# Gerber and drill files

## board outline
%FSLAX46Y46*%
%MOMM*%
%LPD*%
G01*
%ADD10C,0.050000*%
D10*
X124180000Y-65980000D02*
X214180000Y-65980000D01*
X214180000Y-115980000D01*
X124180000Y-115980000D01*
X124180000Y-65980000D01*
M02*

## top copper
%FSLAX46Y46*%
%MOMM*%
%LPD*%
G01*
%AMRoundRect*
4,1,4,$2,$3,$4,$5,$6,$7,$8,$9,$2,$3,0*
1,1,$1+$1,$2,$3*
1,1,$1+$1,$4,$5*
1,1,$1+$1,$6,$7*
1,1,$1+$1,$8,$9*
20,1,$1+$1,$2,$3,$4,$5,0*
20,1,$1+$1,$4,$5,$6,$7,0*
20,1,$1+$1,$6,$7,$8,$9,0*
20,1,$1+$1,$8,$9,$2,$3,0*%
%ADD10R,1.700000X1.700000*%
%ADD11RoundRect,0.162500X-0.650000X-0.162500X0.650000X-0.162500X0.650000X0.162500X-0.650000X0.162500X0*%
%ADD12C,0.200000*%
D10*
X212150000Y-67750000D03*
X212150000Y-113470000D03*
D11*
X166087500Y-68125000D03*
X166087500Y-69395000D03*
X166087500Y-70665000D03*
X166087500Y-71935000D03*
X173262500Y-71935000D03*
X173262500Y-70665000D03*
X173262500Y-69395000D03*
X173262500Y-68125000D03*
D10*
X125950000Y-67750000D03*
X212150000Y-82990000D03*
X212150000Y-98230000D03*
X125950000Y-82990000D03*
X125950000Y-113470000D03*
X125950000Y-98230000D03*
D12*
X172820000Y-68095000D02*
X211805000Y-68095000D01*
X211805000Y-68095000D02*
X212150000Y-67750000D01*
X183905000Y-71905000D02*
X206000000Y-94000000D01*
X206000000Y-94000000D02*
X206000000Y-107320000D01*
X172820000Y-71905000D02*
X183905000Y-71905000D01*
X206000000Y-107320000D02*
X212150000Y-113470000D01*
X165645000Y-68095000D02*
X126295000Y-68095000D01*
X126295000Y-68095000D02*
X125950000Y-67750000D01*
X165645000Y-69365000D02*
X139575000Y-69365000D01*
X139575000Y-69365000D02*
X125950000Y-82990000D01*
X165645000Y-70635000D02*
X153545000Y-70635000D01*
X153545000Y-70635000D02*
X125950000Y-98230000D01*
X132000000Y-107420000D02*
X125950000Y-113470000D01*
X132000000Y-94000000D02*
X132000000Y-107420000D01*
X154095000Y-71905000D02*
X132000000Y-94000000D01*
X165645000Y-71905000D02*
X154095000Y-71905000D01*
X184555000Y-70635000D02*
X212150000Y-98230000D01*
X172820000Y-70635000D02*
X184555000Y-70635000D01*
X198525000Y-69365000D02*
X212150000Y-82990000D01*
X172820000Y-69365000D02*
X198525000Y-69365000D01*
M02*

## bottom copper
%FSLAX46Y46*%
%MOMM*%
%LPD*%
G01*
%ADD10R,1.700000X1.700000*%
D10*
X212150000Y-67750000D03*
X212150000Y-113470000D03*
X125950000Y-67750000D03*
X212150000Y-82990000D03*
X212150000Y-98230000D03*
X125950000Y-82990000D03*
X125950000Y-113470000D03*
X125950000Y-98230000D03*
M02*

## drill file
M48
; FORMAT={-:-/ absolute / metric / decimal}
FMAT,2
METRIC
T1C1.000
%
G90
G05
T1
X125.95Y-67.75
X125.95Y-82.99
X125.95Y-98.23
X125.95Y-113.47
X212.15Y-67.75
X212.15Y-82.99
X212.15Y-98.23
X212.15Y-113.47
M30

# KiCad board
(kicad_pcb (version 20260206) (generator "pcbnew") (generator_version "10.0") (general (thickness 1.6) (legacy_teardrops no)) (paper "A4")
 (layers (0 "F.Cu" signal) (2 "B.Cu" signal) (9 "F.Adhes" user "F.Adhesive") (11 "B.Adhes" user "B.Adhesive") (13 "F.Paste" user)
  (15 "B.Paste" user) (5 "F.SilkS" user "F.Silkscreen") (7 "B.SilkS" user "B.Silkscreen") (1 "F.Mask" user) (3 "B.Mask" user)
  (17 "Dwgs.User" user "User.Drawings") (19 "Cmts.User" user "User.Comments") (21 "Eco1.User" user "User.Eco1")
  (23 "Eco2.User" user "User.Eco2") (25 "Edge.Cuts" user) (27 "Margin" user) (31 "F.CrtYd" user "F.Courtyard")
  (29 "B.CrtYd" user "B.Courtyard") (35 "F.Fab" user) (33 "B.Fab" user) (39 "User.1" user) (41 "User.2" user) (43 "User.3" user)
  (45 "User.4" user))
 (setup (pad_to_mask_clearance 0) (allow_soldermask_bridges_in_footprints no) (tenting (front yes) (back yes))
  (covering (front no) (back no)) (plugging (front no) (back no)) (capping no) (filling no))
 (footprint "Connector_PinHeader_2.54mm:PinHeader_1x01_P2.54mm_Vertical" (layer "F.Cu") (at 212.15 67.75)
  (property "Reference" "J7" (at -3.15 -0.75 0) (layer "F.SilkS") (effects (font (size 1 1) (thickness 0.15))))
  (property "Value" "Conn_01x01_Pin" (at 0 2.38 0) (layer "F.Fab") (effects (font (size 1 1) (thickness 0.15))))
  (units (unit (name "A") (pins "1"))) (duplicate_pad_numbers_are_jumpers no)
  (pad "1" thru_hole rect (at 0 0) (size 1.7 1.7) (drill 1) (layers "*.Cu" "*.Mask") (remove_unused_layers no) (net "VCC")))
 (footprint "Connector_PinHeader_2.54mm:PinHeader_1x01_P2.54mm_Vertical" (layer "F.Cu") (at 212.15 113.47)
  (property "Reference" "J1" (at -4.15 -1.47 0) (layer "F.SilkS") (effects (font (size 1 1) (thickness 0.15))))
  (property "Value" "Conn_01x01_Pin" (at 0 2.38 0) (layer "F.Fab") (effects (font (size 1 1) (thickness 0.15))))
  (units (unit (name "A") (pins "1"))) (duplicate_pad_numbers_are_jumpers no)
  (pad "1" thru_hole rect (at 0 0) (size 1.7 1.7) (drill 1) (layers "*.Cu" "*.Mask") (remove_unused_layers no) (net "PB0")))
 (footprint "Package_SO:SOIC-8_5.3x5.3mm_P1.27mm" (layer "F.Cu") (at 169.675 70.03)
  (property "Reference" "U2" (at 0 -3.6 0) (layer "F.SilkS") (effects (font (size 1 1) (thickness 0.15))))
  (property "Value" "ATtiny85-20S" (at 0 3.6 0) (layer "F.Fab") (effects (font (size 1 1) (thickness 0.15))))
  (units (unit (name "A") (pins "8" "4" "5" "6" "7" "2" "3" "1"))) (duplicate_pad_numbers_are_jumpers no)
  (pad "1" smd roundrect (at -3.5875 -1.905) (size 1.625 0.65) (layers "F.Cu" "F.Mask" "F.Paste") (roundrect_rratio 0.25) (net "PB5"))
  (pad "2" smd roundrect (at -3.5875 -0.635) (size 1.625 0.65) (layers "F.Cu" "F.Mask" "F.Paste") (roundrect_rratio 0.25) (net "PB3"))
  (pad "3" smd roundrect (at -3.5875 0.635) (size 1.625 0.65) (layers "F.Cu" "F.Mask" "F.Paste") (roundrect_rratio 0.25) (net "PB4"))
  (pad "4" smd roundrect (at -3.5875 1.905) (size 1.625 0.65) (layers "F.Cu" "F.Mask" "F.Paste") (roundrect_rratio 0.25) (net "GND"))
  (pad "5" smd roundrect (at 3.5875 1.905) (size 1.625 0.65) (layers "F.Cu" "F.Mask" "F.Paste") (roundrect_rratio 0.25) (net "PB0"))
  (pad "6" smd roundrect (at 3.5875 0.635) (size 1.625 0.65) (layers "F.Cu" "F.Mask" "F.Paste") (roundrect_rratio 0.25) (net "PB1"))
  (pad "7" smd roundrect (at 3.5875 -0.635) (size 1.625 0.65) (layers "F.Cu" "F.Mask" "F.Paste") (roundrect_rratio 0.25) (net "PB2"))
  (pad "8" smd roundrect (at 3.5875 -1.905) (size 1.625 0.65) (layers "F.Cu" "F.Mask" "F.Paste") (roundrect_rratio 0.25) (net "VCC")))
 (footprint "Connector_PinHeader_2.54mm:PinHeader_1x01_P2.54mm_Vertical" (layer "F.Cu") (at 125.95 67.75)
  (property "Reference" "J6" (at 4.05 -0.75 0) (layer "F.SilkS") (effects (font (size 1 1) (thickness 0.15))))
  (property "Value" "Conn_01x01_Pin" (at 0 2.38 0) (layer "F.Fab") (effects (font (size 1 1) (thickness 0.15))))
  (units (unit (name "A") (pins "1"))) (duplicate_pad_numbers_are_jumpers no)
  (pad "1" thru_hole rect (at 0 0) (size 1.7 1.7) (drill 1) (layers "*.Cu" "*.Mask") (remove_unused_layers no) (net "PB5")))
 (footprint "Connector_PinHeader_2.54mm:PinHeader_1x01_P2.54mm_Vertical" (layer "F.Cu") (at 212.15 82.99)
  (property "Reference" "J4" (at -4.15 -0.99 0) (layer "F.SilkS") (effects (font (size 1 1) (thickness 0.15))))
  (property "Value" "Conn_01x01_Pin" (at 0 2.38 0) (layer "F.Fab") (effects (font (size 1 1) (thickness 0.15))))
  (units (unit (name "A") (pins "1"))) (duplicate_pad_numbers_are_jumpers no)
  (pad "1" thru_hole rect (at 0 0) (size 1.7 1.7) (drill 1) (layers "*.Cu" "*.Mask") (remove_unused_layers no) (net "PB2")))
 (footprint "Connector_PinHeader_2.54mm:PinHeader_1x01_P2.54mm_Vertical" (layer "F.Cu") (at 212.15 98.23)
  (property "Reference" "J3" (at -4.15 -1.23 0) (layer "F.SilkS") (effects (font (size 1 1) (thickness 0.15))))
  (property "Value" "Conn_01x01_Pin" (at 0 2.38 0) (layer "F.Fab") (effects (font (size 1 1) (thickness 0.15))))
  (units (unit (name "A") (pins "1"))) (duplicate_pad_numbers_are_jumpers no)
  (pad "1" thru_hole rect (at 0 0) (size 1.7 1.7) (drill 1) (layers "*.Cu" "*.Mask") (remove_unused_layers no) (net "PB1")))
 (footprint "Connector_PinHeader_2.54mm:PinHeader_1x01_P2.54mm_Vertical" (layer "F.Cu") (at 125.95 82.99)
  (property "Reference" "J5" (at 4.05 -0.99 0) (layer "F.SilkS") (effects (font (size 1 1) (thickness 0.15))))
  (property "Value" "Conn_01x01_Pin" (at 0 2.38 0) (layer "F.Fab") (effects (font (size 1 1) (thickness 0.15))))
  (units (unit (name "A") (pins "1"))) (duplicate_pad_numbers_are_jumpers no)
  (pad "1" thru_hole rect (at 0 0) (size 1.7 1.7) (drill 1) (layers "*.Cu" "*.Mask") (remove_unused_layers no) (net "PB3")))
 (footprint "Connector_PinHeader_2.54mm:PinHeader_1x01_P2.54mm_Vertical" (layer "F.Cu") (at 125.95 113.47)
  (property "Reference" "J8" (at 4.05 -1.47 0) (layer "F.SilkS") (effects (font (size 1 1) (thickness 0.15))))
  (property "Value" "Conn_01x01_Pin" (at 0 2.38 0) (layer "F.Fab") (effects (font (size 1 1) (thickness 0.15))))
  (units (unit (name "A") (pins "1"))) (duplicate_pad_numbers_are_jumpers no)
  (pad "1" thru_hole rect (at 0 0) (size 1.7 1.7) (drill 1) (layers "*.Cu" "*.Mask") (remove_unused_layers no) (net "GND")))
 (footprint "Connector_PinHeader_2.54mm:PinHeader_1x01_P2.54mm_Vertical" (layer "F.Cu") (at 125.95 98.23)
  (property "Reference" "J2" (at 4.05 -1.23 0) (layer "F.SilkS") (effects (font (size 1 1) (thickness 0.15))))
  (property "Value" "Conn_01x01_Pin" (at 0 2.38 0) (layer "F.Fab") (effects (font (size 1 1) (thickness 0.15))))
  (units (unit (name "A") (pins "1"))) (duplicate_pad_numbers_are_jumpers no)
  (pad "1" thru_hole rect (at 0 0) (size 1.7 1.7) (drill 1) (layers "*.Cu" "*.Mask") (remove_unused_layers no) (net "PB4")))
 (gr_rect (start 124.18 65.98) (end 214.18 115.98) (stroke (width 0.05) (type default)) (fill no) (layer "Edge.Cuts"))
 (segment (start 172.82 68.095) (end 211.805 68.095) (width 0.2) (layer "F.Cu") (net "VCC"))
 (segment (start 211.805 68.095) (end 212.15 67.75) (width 0.2) (layer "F.Cu") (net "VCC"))
 (segment (start 183.905 71.905) (end 206 94) (width 0.2) (layer "F.Cu") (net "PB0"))
 (segment (start 206 94) (end 206 107.32) (width 0.2) (layer "F.Cu") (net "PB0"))
 (segment (start 172.82 71.905) (end 183.905 71.905) (width 0.2) (layer "F.Cu") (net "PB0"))
 (segment (start 206 107.32) (end 212.15 113.47) (width 0.2) (layer "F.Cu") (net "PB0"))
 (segment (start 165.645 68.095) (end 126.295 68.095) (width 0.2) (layer "F.Cu") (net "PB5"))
 (segment (start 126.295 68.095) (end 125.95 67.75) (width 0.2) (layer "F.Cu") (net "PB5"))
 (segment (start 165.645 69.365) (end 139.575 69.365) (width 0.2) (layer "F.Cu") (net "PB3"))
 (segment (start 139.575 69.365) (end 125.95 82.99) (width 0.2) (layer "F.Cu") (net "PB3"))
 (segment (start 165.645 70.635) (end 153.545 70.635) (width 0.2) (layer "F.Cu") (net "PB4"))
 (segment (start 153.545 70.635) (end 125.95 98.23) (width 0.2) (layer "F.Cu") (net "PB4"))
 (segment (start 132 107.42) (end 125.95 113.47) (width 0.2) (layer "F.Cu") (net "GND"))
 (segment (start 132 94) (end 132 107.42) (width 0.2) (layer "F.Cu") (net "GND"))
 (segment (start 154.095 71.905) (end 132 94) (width 0.2) (layer "F.Cu") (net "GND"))
 (segment (start 165.645 71.905) (end 154.095 71.905) (width 0.2) (layer "F.Cu") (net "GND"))
 (segment (start 184.555 70.635) (end 212.15 98.23) (width 0.2) (layer "F.Cu") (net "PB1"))
 (segment (start 172.82 70.635) (end 184.555 70.635) (width 0.2) (layer "F.Cu") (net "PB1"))
 (segment (start 198.525 69.365) (end 212.15 82.99) (width 0.2) (layer "F.Cu") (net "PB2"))
 (segment (start 172.82 69.365) (end 198.525 69.365) (width 0.2) (layer "F.Cu") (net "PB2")))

